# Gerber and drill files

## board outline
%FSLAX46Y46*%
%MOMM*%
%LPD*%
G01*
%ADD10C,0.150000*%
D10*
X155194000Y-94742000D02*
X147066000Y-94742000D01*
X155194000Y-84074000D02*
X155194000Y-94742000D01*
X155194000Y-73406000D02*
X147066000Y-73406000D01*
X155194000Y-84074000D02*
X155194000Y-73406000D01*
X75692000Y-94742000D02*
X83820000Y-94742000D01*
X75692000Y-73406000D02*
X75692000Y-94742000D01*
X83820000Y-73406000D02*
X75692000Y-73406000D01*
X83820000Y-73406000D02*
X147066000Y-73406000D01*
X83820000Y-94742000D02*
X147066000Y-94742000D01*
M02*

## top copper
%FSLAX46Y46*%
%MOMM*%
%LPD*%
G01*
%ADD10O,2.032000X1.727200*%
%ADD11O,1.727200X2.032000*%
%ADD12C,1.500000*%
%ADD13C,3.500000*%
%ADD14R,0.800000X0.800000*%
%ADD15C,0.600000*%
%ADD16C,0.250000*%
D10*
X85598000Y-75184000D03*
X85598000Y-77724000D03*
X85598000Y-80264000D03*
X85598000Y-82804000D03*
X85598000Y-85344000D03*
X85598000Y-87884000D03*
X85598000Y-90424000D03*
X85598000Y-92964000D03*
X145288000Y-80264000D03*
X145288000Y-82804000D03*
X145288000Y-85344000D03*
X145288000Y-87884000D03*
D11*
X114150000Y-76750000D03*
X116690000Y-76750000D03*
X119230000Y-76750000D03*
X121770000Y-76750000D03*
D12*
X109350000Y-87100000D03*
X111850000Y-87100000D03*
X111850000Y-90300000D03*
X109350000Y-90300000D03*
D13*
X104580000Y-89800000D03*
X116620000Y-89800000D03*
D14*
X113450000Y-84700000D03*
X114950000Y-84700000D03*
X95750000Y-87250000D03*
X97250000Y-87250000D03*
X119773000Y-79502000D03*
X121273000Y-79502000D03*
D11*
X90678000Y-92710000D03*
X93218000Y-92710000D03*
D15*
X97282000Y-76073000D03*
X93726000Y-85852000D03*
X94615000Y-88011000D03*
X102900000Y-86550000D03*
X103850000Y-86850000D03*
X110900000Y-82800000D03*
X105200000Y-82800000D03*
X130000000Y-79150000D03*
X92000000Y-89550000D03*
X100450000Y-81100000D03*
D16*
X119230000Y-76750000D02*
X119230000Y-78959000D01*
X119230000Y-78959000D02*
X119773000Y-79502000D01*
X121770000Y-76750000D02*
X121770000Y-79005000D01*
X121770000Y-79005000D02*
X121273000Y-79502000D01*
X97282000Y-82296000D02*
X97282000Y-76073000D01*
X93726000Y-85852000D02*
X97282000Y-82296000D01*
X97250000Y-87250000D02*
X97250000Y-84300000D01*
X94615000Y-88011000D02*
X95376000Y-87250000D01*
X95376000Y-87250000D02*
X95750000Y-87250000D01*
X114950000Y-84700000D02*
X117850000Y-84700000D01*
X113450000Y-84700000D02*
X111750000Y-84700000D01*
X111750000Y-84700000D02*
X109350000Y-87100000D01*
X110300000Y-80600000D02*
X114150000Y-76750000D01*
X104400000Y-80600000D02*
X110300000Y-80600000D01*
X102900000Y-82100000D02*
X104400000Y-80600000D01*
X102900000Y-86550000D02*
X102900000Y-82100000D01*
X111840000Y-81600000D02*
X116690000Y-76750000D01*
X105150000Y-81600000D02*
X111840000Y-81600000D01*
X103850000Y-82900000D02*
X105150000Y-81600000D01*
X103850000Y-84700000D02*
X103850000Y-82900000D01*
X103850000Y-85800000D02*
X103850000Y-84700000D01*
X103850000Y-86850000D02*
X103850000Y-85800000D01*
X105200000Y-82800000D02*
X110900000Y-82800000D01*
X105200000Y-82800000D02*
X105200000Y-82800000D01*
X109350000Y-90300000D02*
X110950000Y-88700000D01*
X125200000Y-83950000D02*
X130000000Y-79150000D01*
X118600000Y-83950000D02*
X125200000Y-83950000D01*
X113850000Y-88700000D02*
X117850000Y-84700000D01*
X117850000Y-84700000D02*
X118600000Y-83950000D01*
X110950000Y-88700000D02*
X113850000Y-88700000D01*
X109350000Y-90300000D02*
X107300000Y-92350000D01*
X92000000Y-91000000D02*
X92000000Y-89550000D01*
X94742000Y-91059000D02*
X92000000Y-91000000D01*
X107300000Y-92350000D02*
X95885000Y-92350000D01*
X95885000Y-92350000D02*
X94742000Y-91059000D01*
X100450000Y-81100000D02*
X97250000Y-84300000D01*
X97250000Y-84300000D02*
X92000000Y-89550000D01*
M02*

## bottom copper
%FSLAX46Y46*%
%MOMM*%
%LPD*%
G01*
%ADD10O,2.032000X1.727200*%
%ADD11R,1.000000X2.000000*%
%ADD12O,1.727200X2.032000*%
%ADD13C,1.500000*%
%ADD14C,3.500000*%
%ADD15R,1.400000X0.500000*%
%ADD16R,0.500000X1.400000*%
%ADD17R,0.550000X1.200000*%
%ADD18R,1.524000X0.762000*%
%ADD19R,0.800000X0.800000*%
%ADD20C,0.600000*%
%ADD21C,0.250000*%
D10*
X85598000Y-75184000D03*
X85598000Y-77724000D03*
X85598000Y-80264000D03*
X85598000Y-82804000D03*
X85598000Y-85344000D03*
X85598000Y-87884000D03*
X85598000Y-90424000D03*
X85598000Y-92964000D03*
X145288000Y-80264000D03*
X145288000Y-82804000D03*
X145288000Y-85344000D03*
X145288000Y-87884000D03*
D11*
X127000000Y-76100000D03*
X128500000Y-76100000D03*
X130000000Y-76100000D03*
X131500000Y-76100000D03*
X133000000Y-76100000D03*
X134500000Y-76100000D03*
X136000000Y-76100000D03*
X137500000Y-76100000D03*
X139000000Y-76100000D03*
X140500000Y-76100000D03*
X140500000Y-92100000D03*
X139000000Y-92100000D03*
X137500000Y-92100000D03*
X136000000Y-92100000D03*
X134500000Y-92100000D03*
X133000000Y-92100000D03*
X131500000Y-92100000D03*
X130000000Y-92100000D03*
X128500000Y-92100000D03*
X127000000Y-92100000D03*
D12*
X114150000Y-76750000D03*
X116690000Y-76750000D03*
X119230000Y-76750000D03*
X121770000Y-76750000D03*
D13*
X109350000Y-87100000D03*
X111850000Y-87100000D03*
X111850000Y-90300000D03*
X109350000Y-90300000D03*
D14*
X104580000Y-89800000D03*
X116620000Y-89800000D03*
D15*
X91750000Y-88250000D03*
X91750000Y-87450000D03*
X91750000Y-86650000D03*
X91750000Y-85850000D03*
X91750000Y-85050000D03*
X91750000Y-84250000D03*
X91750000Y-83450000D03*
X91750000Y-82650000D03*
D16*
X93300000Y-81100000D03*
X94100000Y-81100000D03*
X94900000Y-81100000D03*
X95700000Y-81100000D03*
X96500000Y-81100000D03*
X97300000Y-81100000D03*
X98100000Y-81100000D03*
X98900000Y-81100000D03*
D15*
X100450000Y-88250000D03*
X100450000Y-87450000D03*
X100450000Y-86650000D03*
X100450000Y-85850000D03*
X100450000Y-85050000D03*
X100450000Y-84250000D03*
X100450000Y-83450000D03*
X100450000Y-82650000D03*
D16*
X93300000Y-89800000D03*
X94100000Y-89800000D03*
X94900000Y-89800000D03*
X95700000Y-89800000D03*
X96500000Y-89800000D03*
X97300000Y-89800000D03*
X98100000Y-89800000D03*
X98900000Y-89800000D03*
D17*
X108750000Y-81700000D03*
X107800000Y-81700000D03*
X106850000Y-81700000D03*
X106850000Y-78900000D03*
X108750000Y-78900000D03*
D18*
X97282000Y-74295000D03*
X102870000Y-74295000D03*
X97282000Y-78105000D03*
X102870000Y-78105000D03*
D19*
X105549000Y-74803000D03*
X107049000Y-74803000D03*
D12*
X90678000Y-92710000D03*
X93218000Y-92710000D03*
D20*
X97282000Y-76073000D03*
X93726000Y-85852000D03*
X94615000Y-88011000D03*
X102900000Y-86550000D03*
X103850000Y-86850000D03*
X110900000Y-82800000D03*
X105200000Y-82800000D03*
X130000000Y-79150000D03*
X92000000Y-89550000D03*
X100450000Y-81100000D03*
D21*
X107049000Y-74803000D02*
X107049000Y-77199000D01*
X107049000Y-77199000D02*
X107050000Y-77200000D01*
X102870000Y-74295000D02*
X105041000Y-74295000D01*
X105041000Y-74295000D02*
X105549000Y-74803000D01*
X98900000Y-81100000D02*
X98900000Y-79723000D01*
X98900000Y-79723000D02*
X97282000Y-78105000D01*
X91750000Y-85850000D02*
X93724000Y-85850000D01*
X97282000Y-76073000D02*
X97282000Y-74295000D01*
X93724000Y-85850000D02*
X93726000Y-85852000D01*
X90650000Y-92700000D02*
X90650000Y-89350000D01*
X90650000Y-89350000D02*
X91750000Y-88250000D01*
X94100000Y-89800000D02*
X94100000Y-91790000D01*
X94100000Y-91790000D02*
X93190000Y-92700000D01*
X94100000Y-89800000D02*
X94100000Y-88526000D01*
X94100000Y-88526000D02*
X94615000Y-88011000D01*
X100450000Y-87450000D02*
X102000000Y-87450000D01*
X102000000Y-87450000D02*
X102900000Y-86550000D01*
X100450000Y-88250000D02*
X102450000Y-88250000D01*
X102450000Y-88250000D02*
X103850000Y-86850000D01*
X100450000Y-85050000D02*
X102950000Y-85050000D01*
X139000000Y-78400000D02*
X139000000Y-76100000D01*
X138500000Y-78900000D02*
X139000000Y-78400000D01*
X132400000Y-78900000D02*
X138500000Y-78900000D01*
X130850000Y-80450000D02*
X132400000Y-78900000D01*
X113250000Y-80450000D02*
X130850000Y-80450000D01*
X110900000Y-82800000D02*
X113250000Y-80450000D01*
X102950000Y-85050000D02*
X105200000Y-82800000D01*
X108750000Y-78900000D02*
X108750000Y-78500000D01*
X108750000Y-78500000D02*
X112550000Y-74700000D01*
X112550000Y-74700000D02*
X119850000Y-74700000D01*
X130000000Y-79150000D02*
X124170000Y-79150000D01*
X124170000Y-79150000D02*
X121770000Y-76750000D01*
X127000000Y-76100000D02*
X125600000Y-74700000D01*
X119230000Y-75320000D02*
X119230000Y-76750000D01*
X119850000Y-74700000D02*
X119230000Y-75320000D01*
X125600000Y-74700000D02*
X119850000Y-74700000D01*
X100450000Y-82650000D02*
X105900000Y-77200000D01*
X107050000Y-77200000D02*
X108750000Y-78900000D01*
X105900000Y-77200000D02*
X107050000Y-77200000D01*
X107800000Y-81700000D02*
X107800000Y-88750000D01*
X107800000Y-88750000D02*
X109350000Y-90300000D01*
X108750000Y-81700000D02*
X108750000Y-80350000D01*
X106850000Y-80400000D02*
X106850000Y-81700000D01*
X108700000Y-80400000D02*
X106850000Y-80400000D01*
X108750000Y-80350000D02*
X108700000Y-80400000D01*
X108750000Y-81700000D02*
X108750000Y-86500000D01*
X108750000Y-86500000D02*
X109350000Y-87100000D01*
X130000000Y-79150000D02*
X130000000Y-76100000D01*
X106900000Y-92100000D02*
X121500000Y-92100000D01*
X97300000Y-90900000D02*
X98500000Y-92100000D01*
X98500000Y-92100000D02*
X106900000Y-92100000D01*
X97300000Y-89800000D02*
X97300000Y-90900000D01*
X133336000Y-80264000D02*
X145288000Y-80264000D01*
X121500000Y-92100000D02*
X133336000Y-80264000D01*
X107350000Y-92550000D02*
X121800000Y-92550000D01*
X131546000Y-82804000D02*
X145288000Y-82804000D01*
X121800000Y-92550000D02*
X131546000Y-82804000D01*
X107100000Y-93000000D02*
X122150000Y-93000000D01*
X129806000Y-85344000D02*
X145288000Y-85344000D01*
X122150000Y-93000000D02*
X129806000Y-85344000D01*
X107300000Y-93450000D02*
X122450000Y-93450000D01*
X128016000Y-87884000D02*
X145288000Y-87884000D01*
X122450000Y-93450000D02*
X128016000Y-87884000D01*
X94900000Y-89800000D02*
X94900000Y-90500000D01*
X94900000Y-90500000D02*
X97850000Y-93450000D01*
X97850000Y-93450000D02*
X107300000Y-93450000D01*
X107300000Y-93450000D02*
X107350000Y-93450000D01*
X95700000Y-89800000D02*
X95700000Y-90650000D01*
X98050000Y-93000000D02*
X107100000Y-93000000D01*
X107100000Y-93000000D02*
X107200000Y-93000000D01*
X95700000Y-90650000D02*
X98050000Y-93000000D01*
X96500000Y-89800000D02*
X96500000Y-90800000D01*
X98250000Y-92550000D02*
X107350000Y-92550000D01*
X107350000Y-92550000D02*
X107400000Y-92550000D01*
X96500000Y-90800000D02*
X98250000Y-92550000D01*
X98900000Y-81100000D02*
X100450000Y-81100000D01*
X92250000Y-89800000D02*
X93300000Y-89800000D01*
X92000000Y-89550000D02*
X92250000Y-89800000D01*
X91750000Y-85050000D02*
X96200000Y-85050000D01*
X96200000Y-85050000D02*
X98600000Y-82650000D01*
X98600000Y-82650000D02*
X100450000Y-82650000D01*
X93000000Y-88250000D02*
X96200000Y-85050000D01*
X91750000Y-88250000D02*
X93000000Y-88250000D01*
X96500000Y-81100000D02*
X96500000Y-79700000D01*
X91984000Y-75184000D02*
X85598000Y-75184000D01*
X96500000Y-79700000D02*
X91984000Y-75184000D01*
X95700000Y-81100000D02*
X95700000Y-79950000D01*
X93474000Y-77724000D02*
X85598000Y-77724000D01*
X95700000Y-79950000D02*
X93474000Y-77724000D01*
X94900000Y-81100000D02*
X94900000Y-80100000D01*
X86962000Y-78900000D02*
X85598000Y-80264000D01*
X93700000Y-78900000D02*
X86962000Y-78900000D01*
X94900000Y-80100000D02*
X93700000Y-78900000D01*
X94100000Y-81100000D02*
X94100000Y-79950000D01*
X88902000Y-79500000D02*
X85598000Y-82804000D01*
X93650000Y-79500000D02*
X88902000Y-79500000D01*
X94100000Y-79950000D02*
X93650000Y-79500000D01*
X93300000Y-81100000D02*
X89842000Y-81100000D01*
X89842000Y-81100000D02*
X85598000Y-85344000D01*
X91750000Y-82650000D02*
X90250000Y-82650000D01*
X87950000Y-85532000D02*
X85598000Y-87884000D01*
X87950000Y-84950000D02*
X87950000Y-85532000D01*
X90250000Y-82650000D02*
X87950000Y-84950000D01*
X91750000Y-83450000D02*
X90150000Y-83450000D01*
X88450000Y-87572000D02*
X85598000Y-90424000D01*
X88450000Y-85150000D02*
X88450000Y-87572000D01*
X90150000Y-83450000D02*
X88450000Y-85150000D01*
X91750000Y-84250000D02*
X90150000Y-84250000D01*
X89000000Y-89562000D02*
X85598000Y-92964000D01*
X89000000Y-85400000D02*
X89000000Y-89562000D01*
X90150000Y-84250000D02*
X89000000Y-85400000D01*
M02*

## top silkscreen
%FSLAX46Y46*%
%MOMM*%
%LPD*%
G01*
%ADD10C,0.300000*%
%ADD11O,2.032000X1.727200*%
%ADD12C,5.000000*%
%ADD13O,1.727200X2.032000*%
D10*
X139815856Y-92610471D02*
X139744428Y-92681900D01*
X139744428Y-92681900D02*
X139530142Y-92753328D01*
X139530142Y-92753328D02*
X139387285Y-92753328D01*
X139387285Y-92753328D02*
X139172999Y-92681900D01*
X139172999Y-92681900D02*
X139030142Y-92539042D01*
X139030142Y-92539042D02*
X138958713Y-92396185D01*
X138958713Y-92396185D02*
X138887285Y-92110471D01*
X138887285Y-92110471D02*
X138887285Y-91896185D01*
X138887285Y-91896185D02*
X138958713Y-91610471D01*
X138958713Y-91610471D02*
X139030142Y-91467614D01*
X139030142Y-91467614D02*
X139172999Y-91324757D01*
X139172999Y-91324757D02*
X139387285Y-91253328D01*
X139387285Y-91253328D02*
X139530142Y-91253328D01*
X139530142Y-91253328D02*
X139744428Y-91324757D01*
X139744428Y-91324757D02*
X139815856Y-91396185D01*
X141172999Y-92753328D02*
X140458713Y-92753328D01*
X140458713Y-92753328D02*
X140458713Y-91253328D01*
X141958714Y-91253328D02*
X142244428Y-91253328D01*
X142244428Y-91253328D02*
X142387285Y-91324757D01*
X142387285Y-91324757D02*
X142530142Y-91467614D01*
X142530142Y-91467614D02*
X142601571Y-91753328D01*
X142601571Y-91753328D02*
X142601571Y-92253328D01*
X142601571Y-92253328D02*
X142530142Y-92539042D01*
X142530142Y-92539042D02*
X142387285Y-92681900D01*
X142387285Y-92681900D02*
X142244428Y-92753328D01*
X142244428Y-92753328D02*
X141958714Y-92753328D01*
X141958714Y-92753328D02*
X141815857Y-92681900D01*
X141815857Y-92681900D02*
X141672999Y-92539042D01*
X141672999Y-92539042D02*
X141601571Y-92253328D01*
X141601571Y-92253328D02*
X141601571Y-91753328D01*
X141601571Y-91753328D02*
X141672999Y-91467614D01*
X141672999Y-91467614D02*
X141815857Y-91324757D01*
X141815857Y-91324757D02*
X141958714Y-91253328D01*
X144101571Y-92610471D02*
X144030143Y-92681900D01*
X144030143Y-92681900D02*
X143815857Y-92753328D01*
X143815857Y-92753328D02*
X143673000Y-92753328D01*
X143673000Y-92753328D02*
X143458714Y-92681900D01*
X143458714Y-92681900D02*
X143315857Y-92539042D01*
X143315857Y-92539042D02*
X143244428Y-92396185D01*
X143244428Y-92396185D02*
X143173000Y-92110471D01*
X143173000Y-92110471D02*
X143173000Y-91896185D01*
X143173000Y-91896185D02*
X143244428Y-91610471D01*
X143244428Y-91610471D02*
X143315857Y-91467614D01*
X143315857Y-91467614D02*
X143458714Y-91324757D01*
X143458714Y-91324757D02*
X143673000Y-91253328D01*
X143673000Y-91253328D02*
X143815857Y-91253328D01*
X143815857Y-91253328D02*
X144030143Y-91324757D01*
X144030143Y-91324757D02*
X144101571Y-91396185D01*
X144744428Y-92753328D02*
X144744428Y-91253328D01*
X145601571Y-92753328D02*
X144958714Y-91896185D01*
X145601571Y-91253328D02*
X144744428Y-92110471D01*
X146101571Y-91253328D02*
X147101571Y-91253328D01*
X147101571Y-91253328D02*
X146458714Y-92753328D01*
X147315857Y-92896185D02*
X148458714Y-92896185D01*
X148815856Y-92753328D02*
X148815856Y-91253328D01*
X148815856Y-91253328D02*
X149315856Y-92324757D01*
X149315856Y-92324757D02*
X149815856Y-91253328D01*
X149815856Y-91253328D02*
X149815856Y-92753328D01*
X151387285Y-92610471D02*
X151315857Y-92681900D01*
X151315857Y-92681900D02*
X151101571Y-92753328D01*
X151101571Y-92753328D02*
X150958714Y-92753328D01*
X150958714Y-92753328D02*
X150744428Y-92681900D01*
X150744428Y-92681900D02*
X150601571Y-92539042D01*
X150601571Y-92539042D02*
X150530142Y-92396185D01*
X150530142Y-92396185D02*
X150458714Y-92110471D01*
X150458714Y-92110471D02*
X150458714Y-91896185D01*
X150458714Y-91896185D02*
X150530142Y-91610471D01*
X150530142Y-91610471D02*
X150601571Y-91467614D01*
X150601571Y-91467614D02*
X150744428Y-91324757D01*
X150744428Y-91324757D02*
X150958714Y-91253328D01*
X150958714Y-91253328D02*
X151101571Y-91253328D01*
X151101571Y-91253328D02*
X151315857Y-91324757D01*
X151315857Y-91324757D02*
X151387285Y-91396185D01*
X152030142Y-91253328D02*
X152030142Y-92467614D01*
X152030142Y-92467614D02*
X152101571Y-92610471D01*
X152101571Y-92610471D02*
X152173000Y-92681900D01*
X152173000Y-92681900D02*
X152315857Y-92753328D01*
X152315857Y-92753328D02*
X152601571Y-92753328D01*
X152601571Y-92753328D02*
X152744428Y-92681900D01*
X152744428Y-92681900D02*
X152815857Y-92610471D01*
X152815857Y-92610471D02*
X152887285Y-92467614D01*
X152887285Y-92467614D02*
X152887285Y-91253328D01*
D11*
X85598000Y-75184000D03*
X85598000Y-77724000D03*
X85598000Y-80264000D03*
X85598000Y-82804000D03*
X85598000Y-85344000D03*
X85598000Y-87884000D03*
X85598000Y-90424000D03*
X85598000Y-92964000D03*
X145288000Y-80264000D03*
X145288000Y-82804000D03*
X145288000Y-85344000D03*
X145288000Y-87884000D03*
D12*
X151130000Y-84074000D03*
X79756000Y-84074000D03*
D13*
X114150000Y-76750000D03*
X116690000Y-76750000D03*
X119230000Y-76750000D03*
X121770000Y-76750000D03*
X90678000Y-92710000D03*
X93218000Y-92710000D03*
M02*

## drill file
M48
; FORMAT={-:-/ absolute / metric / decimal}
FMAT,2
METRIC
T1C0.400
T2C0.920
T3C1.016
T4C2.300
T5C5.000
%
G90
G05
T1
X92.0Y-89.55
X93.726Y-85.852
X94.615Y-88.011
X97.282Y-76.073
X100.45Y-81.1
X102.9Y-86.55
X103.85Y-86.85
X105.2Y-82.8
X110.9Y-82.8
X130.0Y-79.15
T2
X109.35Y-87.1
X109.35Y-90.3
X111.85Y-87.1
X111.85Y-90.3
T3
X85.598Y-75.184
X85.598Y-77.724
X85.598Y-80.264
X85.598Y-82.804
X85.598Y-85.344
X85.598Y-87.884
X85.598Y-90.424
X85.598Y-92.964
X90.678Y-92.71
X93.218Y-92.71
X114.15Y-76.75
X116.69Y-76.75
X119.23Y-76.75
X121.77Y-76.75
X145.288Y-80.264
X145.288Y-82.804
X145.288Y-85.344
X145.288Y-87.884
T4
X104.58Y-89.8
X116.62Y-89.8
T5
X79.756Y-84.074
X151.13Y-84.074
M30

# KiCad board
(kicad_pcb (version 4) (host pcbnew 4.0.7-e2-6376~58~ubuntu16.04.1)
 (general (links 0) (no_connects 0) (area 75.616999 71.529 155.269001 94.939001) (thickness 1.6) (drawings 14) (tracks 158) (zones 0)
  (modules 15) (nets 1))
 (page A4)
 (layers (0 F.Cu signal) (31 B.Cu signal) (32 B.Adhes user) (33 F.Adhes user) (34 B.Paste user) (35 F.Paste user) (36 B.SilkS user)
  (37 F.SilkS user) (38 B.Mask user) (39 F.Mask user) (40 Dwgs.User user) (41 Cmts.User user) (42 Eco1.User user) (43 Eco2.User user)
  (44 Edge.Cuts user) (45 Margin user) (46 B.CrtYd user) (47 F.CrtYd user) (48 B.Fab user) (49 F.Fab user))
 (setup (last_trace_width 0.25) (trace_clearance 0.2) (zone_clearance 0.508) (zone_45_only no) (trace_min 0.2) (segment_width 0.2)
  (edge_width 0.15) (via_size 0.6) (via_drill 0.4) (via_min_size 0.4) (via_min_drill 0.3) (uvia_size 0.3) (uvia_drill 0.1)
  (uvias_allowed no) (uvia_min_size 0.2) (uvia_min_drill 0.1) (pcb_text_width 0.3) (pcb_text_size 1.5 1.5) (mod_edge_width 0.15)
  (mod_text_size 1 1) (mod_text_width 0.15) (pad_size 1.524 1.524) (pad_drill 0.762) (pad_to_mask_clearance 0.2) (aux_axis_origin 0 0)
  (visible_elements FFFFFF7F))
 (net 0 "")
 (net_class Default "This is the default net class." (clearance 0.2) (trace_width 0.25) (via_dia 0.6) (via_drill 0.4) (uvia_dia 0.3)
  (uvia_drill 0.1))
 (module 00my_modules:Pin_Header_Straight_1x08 (layer F.Cu) (at 85.598 75.184)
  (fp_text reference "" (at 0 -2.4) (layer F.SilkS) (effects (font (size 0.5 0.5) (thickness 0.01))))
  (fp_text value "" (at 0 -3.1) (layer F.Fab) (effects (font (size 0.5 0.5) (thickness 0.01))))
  (pad 1 thru_hole oval (at 0 0) (size 2.032 1.7272) (drill 1.016) (layers *.Cu *.Mask F.SilkS))
  (pad 2 thru_hole oval (at 0 2.54) (size 2.032 1.7272) (drill 1.016) (layers *.Cu *.Mask F.SilkS))
  (pad 3 thru_hole oval (at 0 5.08) (size 2.032 1.7272) (drill 1.016) (layers *.Cu *.Mask F.SilkS))
  (pad 4 thru_hole oval (at 0 7.62) (size 2.032 1.7272) (drill 1.016) (layers *.Cu *.Mask F.SilkS))
  (pad 5 thru_hole oval (at 0 10.16) (size 2.032 1.7272) (drill 1.016) (layers *.Cu *.Mask F.SilkS))
  (pad 6 thru_hole oval (at 0 12.7) (size 2.032 1.7272) (drill 1.016) (layers *.Cu *.Mask F.SilkS))
  (pad 7 thru_hole oval (at 0 15.24) (size 2.032 1.7272) (drill 1.016) (layers *.Cu *.Mask F.SilkS))
  (pad 8 thru_hole oval (at 0 17.78) (size 2.032 1.7272) (drill 1.016) (layers *.Cu *.Mask F.SilkS)))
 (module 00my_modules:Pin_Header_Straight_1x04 (layer F.Cu) (at 145.288 80.264)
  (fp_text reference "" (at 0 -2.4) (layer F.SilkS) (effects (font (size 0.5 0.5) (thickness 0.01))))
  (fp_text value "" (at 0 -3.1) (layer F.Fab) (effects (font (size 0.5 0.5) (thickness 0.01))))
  (pad 1 thru_hole oval (at 0 0) (size 2.032 1.7272) (drill 1.016) (layers *.Cu *.Mask F.SilkS))
  (pad 2 thru_hole oval (at 0 2.54) (size 2.032 1.7272) (drill 1.016) (layers *.Cu *.Mask F.SilkS))
  (pad 3 thru_hole oval (at 0 5.08) (size 2.032 1.7272) (drill 1.016) (layers *.Cu *.Mask F.SilkS))
  (pad 4 thru_hole oval (at 0 7.62) (size 2.032 1.7272) (drill 1.016) (layers *.Cu *.Mask F.SilkS)))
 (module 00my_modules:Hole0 (layer F.Cu) (at 151.13 84.074)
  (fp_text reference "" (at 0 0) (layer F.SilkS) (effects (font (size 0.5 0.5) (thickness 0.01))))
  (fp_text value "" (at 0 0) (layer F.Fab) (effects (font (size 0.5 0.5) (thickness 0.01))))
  (pad "" np_thru_hole circle (at 0 0) (size 5 5) (drill 5) (layers *.Cu *.Mask F.SilkS)))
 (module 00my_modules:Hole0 (layer F.Cu) (at 79.756 84.074)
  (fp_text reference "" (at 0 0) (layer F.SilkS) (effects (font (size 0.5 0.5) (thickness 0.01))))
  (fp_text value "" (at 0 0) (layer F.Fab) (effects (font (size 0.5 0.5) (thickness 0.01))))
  (pad "" np_thru_hole circle (at 0 0) (size 5 5) (drill 5) (layers *.Cu *.Mask F.SilkS)))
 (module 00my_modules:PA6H (layer B.Cu) (at 133.75 84.1 270)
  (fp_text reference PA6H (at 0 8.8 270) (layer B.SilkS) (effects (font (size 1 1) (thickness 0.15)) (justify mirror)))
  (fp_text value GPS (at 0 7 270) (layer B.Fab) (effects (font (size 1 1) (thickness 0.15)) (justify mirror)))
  (pad VCC smd rect (at -8 6.75 270) (size 2 1) (layers B.Cu B.Paste B.Mask))
  (pad 2 smd rect (at -8 5.25 270) (size 2 1) (layers B.Cu B.Paste B.Mask))
  (pad GND smd rect (at -8 3.75 270) (size 2 1) (layers B.Cu B.Paste B.Mask))
  (pad 4 smd rect (at -8 2.25 270) (size 2 1) (layers B.Cu B.Paste B.Mask))
  (pad 5 smd rect (at -8 0.75 270) (size 2 1) (layers B.Cu B.Paste B.Mask))
  (pad 6 smd rect (at -8 -0.75 270) (size 2 1) (layers B.Cu B.Paste B.Mask))
  (pad 7 smd rect (at -8 -2.25 270) (size 2 1) (layers B.Cu B.Paste B.Mask))
  (pad 8 smd rect (at -8 -3.75 270) (size 2 1) (layers B.Cu B.Paste B.Mask))
  (pad TX smd rect (at -8 -5.25 270) (size 2 1) (layers B.Cu B.Paste B.Mask))
  (pad RX smd rect (at -8 -6.75 270) (size 2 1) (layers B.Cu B.Paste B.Mask))
  (pad 11 smd rect (at 8 -6.75 270) (size 2 1) (layers B.Cu B.Paste B.Mask))
  (pad 12 smd rect (at 8 -5.25 270) (size 2 1) (layers B.Cu B.Paste B.Mask))
  (pad 13 smd rect (at 8 -3.75 270) (size 2 1) (layers B.Cu B.Paste B.Mask))
  (pad 14 smd rect (at 8 -2.25 270) (size 2 1) (layers B.Cu B.Paste B.Mask))
  (pad 15 smd rect (at 8 -0.75 270) (size 2 1) (layers B.Cu B.Paste B.Mask))
  (pad 16 smd rect (at 8 0.75 270) (size 2 1) (layers B.Cu B.Paste B.Mask))
  (pad 17 smd rect (at 8 2.25 270) (size 2 1) (layers B.Cu B.Paste B.Mask))
  (pad 18 smd rect (at 8 3.75 270) (size 2 1) (layers B.Cu B.Paste B.Mask))
  (pad 19 smd rect (at 8 5.25 270) (size 2 1) (layers B.Cu B.Paste B.Mask))
  (pad 20 smd rect (at 8 6.75 270) (size 2 1) (layers B.Cu B.Paste B.Mask)))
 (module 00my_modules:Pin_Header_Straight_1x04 (layer F.Cu) (at 114.15 76.75 90)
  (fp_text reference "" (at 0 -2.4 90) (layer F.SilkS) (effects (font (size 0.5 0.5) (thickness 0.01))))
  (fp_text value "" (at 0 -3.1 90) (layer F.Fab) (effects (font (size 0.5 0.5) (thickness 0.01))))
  (pad 1 thru_hole oval (at 0 0 90) (size 2.032 1.7272) (drill 1.016) (layers *.Cu *.Mask F.SilkS))
  (pad 2 thru_hole oval (at 0 2.54 90) (size 2.032 1.7272) (drill 1.016) (layers *.Cu *.Mask F.SilkS))
  (pad 3 thru_hole oval (at 0 5.08 90) (size 2.032 1.7272) (drill 1.016) (layers *.Cu *.Mask F.SilkS))
  (pad 4 thru_hole oval (at 0 7.62 90) (size 2.032 1.7272) (drill 1.016) (layers *.Cu *.Mask F.SilkS)))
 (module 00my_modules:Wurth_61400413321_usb (layer B.Cu) (at 110.6 89.8 180)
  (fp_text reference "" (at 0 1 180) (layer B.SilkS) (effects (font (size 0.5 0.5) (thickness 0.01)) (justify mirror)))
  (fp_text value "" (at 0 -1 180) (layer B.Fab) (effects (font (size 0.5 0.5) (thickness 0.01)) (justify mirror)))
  (pad V thru_hole circle (at 1.25 2.7 180) (size 1.5 1.5) (drill 0.92) (layers *.Cu *.Mask B.SilkS))
  (pad - thru_hole circle (at -1.25 2.7 180) (size 1.5 1.5) (drill 0.92) (layers *.Cu *.Mask B.SilkS))
  (pad + thru_hole circle (at -1.25 -0.5 180) (size 1.5 1.5) (drill 0.92) (layers *.Cu *.Mask B.SilkS))
  (pad G thru_hole circle (at 1.25 -0.5 180) (size 1.5 1.5) (drill 0.92) (layers *.Cu *.Mask B.SilkS))
  (pad X thru_hole circle (at 6.02 0 180) (size 3.5 3.5) (drill 2.3) (layers *.Cu *.Mask B.SilkS))
  (pad X thru_hole circle (at -6.02 0 180) (size 3.5 3.5) (drill 2.3) (layers *.Cu *.Mask B.SilkS)))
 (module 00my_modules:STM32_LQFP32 (layer B.Cu) (at 96.1 85.45)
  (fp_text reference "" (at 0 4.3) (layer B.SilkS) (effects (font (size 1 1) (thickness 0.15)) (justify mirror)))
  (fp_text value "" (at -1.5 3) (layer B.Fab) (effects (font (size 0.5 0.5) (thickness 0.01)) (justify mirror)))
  (pad 3.3 smd rect (at -4.35 2.8) (size 1.4 0.5) (layers B.Cu B.Paste B.Mask))
  (pad PF0 smd rect (at -4.35 2) (size 1.4 0.5) (layers B.Cu B.Paste B.Mask))
  (pad PF1 smd rect (at -4.35 1.2) (size 1.4 0.5) (layers B.Cu B.Paste B.Mask))
  (pad RST smd rect (at -4.35 0.4) (size 1.4 0.5) (layers B.Cu B.Paste B.Mask))
  (pad 3.3 smd rect (at -4.35 -0.4) (size 1.4 0.5) (layers B.Cu B.Paste B.Mask))
  (pad PA0 smd rect (at -4.35 -1.2) (size 1.4 0.5) (layers B.Cu B.Paste B.Mask))
  (pad PA1 smd rect (at -4.35 -2) (size 1.4 0.5) (layers B.Cu B.Paste B.Mask))
  (pad PA2 smd rect (at -4.35 -2.8) (size 1.4 0.5) (layers B.Cu B.Paste B.Mask))
  (pad PA3 smd rect (at -2.8 -4.35 270) (size 1.4 0.5) (layers B.Cu B.Paste B.Mask))
  (pad PA4 smd rect (at -2 -4.35 270) (size 1.4 0.5) (layers B.Cu B.Paste B.Mask))
  (pad PA5 smd rect (at -1.2 -4.35 270) (size 1.4 0.5) (layers B.Cu B.Paste B.Mask))
  (pad PA6 smd rect (at -0.4 -4.35 270) (size 1.4 0.5) (layers B.Cu B.Paste B.Mask))
  (pad PA7 smd rect (at 0.4 -4.35 270) (size 1.4 0.5) (layers B.Cu B.Paste B.Mask))
  (pad PB0 smd rect (at 1.2 -4.35 270) (size 1.4 0.5) (layers B.Cu B.Paste B.Mask))
  (pad PB1 smd rect (at 2 -4.35 270) (size 1.4 0.5) (layers B.Cu B.Paste B.Mask))
  (pad GND smd rect (at 2.8 -4.35 270) (size 1.4 0.5) (layers B.Cu B.Paste B.Mask))
  (pad PA14 smd rect (at 4.35 2.8) (size 1.4 0.5) (layers B.Cu B.Paste B.Mask))
  (pad PA13 smd rect (at 4.35 2) (size 1.4 0.5) (layers B.Cu B.Paste B.Mask))
  (pad PA12 smd rect (at 4.35 1.2) (size 1.4 0.5) (layers B.Cu B.Paste B.Mask))
  (pad PA11 smd rect (at 4.35 0.4) (size 1.4 0.5) (layers B.Cu B.Paste B.Mask))
  (pad PA10 smd rect (at 4.35 -0.4) (size 1.4 0.5) (layers B.Cu B.Paste B.Mask))
  (pad PA9 smd rect (at 4.35 -1.2) (size 1.4 0.5) (layers B.Cu B.Paste B.Mask))
  (pad PA8 smd rect (at 4.35 -2) (size 1.4 0.5) (layers B.Cu B.Paste B.Mask))
  (pad 3.3 smd rect (at 4.35 -2.8) (size 1.4 0.5) (layers B.Cu B.Paste B.Mask))
  (pad GND smd rect (at -2.8 4.35 270) (size 1.4 0.5) (layers B.Cu B.Paste B.Mask))
  (pad BOOT smd rect (at -2 4.35 270) (size 1.4 0.5) (layers B.Cu B.Paste B.Mask))
  (pad PB7 smd rect (at -1.2 4.35 270) (size 1.4 0.5) (layers B.Cu B.Paste B.Mask))
  (pad PB6 smd rect (at -0.4 4.35 270) (size 1.4 0.5) (layers B.Cu B.Paste B.Mask))
  (pad PB5 smd rect (at 0.4 4.35 270) (size 1.4 0.5) (layers B.Cu B.Paste B.Mask))
  (pad PB4 smd rect (at 1.2 4.35 270) (size 1.4 0.5) (layers B.Cu B.Paste B.Mask))
  (pad PB3 smd rect (at 2 4.35 270) (size 1.4 0.5) (layers B.Cu B.Paste B.Mask))
  (pad PA15 smd rect (at 2.8 4.35 270) (size 1.4 0.5) (layers B.Cu B.Paste B.Mask)))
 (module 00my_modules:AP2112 (layer B.Cu) (at 107.8 80.3 90)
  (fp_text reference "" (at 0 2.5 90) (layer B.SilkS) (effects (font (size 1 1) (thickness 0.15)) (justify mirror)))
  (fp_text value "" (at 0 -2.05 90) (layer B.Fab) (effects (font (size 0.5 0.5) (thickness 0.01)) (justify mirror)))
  (pad VIN smd rect (at -1.4 0.95 90) (size 1.2 0.55) (layers B.Cu B.Paste B.Mask))
  (pad GND smd rect (at -1.4 0 90) (size 1.2 0.55) (layers B.Cu B.Paste B.Mask))
  (pad EN smd rect (at -1.4 -0.95 90) (size 1.2 0.55) (layers B.Cu B.Paste B.Mask))
  (pad NC smd rect (at 1.4 -0.95 90) (size 1.2 0.55) (layers B.Cu B.Paste B.Mask))
  (pad VOUT smd rect (at 1.4 0.95 90) (size 1.2 0.55) (layers B.Cu B.Paste B.Mask)))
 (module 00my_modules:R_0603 (layer F.Cu) (at 114.2 84.7)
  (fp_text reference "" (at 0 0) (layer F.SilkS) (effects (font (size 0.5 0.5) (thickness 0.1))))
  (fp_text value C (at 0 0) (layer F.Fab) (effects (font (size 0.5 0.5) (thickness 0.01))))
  (pad 1 smd rect (at -0.75 0) (size 0.8 0.8) (layers F.Cu F.Paste F.Mask))
  (pad 2 smd rect (at 0.75 0) (size 0.8 0.8) (layers F.Cu F.Paste F.Mask)))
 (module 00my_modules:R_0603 (layer F.Cu) (at 96.5 87.25)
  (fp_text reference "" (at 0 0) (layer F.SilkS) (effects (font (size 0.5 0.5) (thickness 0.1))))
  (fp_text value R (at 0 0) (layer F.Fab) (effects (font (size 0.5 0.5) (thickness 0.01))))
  (pad 1 smd rect (at -0.75 0) (size 0.8 0.8) (layers F.Cu F.Paste F.Mask))
  (pad 2 smd rect (at 0.75 0) (size 0.8 0.8) (layers F.Cu F.Paste F.Mask)))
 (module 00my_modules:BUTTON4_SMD (layer B.Cu) (at 100.076 76.2)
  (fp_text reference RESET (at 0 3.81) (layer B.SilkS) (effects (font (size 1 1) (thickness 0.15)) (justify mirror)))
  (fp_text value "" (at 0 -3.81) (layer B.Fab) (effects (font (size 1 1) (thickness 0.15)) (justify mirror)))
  (pad 1 smd rect (at -2.794 -1.905) (size 1.524 0.762) (layers B.Cu B.Paste B.Mask))
  (pad 2 smd rect (at 2.794 -1.905) (size 1.524 0.762) (layers B.Cu B.Paste B.Mask))
  (pad 3 smd rect (at -2.794 1.905) (size 1.524 0.762) (layers B.Cu B.Paste B.Mask))
  (pad 4 smd rect (at 2.794 1.905) (size 1.524 0.762) (layers B.Cu B.Paste B.Mask)))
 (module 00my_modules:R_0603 (layer B.Cu) (at 106.299 74.803)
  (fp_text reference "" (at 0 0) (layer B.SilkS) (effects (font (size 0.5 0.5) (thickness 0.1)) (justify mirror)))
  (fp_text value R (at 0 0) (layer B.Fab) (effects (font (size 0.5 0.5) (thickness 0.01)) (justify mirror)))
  (pad 1 smd rect (at -0.75 0) (size 0.8 0.8) (layers B.Cu B.Paste B.Mask))
  (pad 2 smd rect (at 0.75 0) (size 0.8 0.8) (layers B.Cu B.Paste B.Mask)))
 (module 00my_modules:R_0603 (layer F.Cu) (at 120.523 79.502)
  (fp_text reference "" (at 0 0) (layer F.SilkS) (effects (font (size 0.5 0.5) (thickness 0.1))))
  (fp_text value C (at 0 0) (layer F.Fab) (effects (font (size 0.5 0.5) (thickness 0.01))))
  (pad 1 smd rect (at -0.75 0) (size 0.8 0.8) (layers F.Cu F.Paste F.Mask))
  (pad 2 smd rect (at 0.75 0) (size 0.8 0.8) (layers F.Cu F.Paste F.Mask)))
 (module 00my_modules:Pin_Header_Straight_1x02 (layer F.Cu) (at 90.678 92.71 90)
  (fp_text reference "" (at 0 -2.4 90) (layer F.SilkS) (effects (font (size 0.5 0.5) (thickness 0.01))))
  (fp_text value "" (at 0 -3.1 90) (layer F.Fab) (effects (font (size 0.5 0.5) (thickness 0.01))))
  (pad 1 thru_hole oval (at 0 0 90) (size 2.032 1.7272) (drill 1.016) (layers *.Cu *.Mask F.SilkS))
  (pad 2 thru_hole oval (at 0 2.54 90) (size 2.032 1.7272) (drill 1.016) (layers *.Cu *.Mask F.SilkS)))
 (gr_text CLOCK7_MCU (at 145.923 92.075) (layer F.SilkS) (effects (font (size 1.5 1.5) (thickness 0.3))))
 (gr_line (start 155.194 94.742) (end 147.066 94.742) (angle 90) (layer Edge.Cuts) (width 0.15))
 (gr_line (start 155.194 84.074) (end 155.194 94.742) (angle 90) (layer Edge.Cuts) (width 0.15))
 (gr_line (start 155.194 73.406) (end 147.066 73.406) (angle 90) (layer Edge.Cuts) (width 0.15))
 (gr_line (start 155.194 84.074) (end 155.194 73.406) (angle 90) (layer Edge.Cuts) (width 0.15))
 (gr_line (start 75.692 94.742) (end 83.82 94.742) (angle 90) (layer Edge.Cuts) (width 0.15))
 (gr_line (start 75.692 73.406) (end 75.692 94.742) (angle 90) (layer Edge.Cuts) (width 0.15))
 (gr_line (start 83.82 73.406) (end 75.692 73.406) (angle 90) (layer Edge.Cuts) (width 0.15))
 (gr_line (start 83.82 73.406) (end 147.066 73.406) (angle 90) (layer Edge.Cuts) (width 0.15))
 (gr_line (start 83.82 94.742) (end 147.066 94.742) (angle 90) (layer Edge.Cuts) (width 0.15))
 (segment (start 119.23 76.75) (end 119.23 78.959) (width 0.25) (layer F.Cu) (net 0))
 (segment (start 119.23 78.959) (end 119.773 79.502) (width 0.25) (layer F.Cu) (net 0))
 (segment (start 121.77 76.75) (end 121.77 79.005) (width 0.25) (layer F.Cu) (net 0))
 (segment (start 121.77 79.005) (end 121.273 79.502) (width 0.25) (layer F.Cu) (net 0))
 (segment (start 107.049 74.803) (end 107.049 77.199) (width 0.25) (layer B.Cu) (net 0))
 (segment (start 107.049 77.199) (end 107.05 77.2) (width 0.25) (layer B.Cu) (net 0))
 (segment (start 102.87 74.295) (end 105.041 74.295) (width 0.25) (layer B.Cu) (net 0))
 (segment (start 105.041 74.295) (end 105.549 74.803) (width 0.25) (layer B.Cu) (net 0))
 (segment (start 98.9 81.1) (end 98.9 79.723) (width 0.25) (layer B.Cu) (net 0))
 (segment (start 98.9 79.723) (end 97.282 78.105) (width 0.25) (layer B.Cu) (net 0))
 (segment (start 91.75 85.85) (end 93.724 85.85) (width 0.25) (layer B.Cu) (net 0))
 (segment (start 97.282 76.073) (end 97.282 74.295) (width 0.25) (layer B.Cu) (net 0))
 (via (at 97.282 76.073) (size 0.6) (drill 0.4) (layers F.Cu B.Cu) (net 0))
 (segment (start 97.282 82.296) (end 97.282 76.073) (width 0.25) (layer F.Cu) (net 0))
 (segment (start 93.726 85.852) (end 97.282 82.296) (width 0.25) (layer F.Cu) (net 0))
 (via (at 93.726 85.852) (size 0.6) (drill 0.4) (layers F.Cu B.Cu) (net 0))
 (segment (start 93.724 85.85) (end 93.726 85.852) (width 0.25) (layer B.Cu) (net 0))
 (segment (start 90.65 92.7) (end 90.65 89.35) (width 0.25) (layer B.Cu) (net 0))
 (segment (start 90.65 89.35) (end 91.75 88.25) (width 0.25) (layer B.Cu) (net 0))
 (segment (start 94.1 89.8) (end 94.1 91.79) (width 0.25) (layer B.Cu) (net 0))
 (segment (start 94.1 91.79) (end 93.19 92.7) (width 0.25) (layer B.Cu) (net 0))
 (segment (start 97.25 87.25) (end 97.25 84.3) (width 0.25) (layer F.Cu) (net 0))
 (segment (start 94.1 89.8) (end 94.1 88.526) (width 0.25) (layer B.Cu) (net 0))
 (segment (start 94.615 88.011) (end 95.376 87.25) (width 0.25) (layer F.Cu) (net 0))
 (via (at 94.615 88.011) (size 0.6) (drill 0.4) (layers F.Cu B.Cu) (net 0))
 (segment (start 94.1 88.526) (end 94.615 88.011) (width 0.25) (layer B.Cu) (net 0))
 (segment (start 95.376 87.25) (end 95.75 87.25) (width 0.25) (layer F.Cu) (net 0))
 (segment (start 114.95 84.7) (end 117.85 84.7) (width 0.25) (layer F.Cu) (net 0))
 (segment (start 113.45 84.7) (end 111.75 84.7) (width 0.25) (layer F.Cu) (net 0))
 (segment (start 111.75 84.7) (end 109.35 87.1) (width 0.25) (layer F.Cu) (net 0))
 (segment (start 100.45 87.45) (end 102 87.45) (width 0.25) (layer B.Cu) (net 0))
 (segment (start 110.3 80.6) (end 114.15 76.75) (width 0.25) (layer F.Cu) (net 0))
 (segment (start 104.4 80.6) (end 110.3 80.6) (width 0.25) (layer F.Cu) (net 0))
 (segment (start 102.9 82.1) (end 104.4 80.6) (width 0.25) (layer F.Cu) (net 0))
 (segment (start 102.9 86.55) (end 102.9 82.1) (width 0.25) (layer F.Cu) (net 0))
 (via (at 102.9 86.55) (size 0.6) (drill 0.4) (layers F.Cu B.Cu) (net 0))
 (segment (start 102 87.45) (end 102.9 86.55) (width 0.25) (layer B.Cu) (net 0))
 (segment (start 100.45 88.25) (end 102.45 88.25) (width 0.25) (layer B.Cu) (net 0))
 (segment (start 111.84 81.6) (end 116.69 76.75) (width 0.25) (layer F.Cu) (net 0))
 (segment (start 105.15 81.6) (end 111.84 81.6) (width 0.25) (layer F.Cu) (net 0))
 (segment (start 103.85 82.9) (end 105.15 81.6) (width 0.25) (layer F.Cu) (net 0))
 (segment (start 103.85 84.7) (end 103.85 82.9) (width 0.25) (layer F.Cu) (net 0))
 (segment (start 103.85 85.8) (end 103.85 84.7) (width 0.25) (layer F.Cu) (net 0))
 (segment (start 103.85 86.85) (end 103.85 85.8) (width 0.25) (layer F.Cu) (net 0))
 (via (at 103.85 86.85) (size 0.6) (drill 0.4) (layers F.Cu B.Cu) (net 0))
 (segment (start 102.45 88.25) (end 103.85 86.85) (width 0.25) (layer B.Cu) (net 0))
 (segment (start 100.45 85.05) (end 102.95 85.05) (width 0.25) (layer B.Cu) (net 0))
 (segment (start 139 78.4) (end 139 76.1) (width 0.25) (layer B.Cu) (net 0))
 (segment (start 138.5 78.9) (end 139 78.4) (width 0.25) (layer B.Cu) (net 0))
 (segment (start 132.4 78.9) (end 138.5 78.9) (width 0.25) (layer B.Cu) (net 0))
 (segment (start 130.85 80.45) (end 132.4 78.9) (width 0.25) (layer B.Cu) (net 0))
 (segment (start 113.25 80.45) (end 130.85 80.45) (width 0.25) (layer B.Cu) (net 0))
 (segment (start 110.9 82.8) (end 113.25 80.45) (width 0.25) (layer B.Cu) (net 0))
 (via (at 110.9 82.8) (size 0.6) (drill 0.4) (layers F.Cu B.Cu) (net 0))
 (segment (start 105.2 82.8) (end 110.9 82.8) (width 0.25) (layer F.Cu) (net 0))
 (segment (start 105.2 82.8) (end 105.2 82.8) (width 0.25) (layer F.Cu) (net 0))
 (via (at 105.2 82.8) (size 0.6) (drill 0.4) (layers F.Cu B.Cu) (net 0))
 (segment (start 102.95 85.05) (end 105.2 82.8) (width 0.25) (layer B.Cu) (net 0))
 (segment (start 108.75 78.9) (end 108.75 78.5) (width 0.25) (layer B.Cu) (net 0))
 (segment (start 108.75 78.5) (end 112.55 74.7) (width 0.25) (layer B.Cu) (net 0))
 (segment (start 112.55 74.7) (end 119.85 74.7) (width 0.25) (layer B.Cu) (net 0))
 (segment (start 130 79.15) (end 124.17 79.15) (width 0.25) (layer B.Cu) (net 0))
 (segment (start 124.17 79.15) (end 121.77 76.75) (width 0.25) (layer B.Cu) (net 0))
 (segment (start 127 76.1) (end 125.6 74.7) (width 0.25) (layer B.Cu) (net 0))
 (segment (start 119.23 75.32) (end 119.23 76.75) (width 0.25) (layer B.Cu) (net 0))
 (segment (start 119.85 74.7) (end 119.23 75.32) (width 0.25) (layer B.Cu) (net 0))
 (segment (start 125.6 74.7) (end 119.85 74.7) (width 0.25) (layer B.Cu) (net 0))
 (segment (start 100.45 82.65) (end 105.9 77.2) (width 0.25) (layer B.Cu) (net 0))
 (segment (start 107.05 77.2) (end 108.75 78.9) (width 0.25) (layer B.Cu) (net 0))
 (segment (start 105.9 77.2) (end 107.05 77.2) (width 0.25) (layer B.Cu) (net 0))
 (segment (start 107.8 81.7) (end 107.8 88.75) (width 0.25) (layer B.Cu) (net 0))
 (segment (start 107.8 88.75) (end 109.35 90.3) (width 0.25) (layer B.Cu) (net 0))
 (segment (start 108.75 81.7) (end 108.75 80.35) (width 0.25) (layer B.Cu) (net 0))
 (segment (start 106.85 80.4) (end 106.85 81.7) (width 0.25) (layer B.Cu) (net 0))
 (segment (start 108.7 80.4) (end 106.85 80.4) (width 0.25) (layer B.Cu) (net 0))
 (segment (start 108.75 80.35) (end 108.7 80.4) (width 0.25) (layer B.Cu) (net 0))
 (segment (start 108.75 81.7) (end 108.75 86.5) (width 0.25) (layer B.Cu) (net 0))
 (segment (start 108.75 86.5) (end 109.35 87.1) (width 0.25) (layer B.Cu) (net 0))
 (segment (start 109.35 90.3) (end 110.95 88.7) (width 0.25) (layer F.Cu) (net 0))
 (segment (start 130 79.15) (end 130 76.1) (width 0.25) (layer B.Cu) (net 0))
 (via (at 130 79.15) (size 0.6) (drill 0.4) (layers F.Cu B.Cu) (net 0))
 (segment (start 125.2 83.95) (end 130 79.15) (width 0.25) (layer F.Cu) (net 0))
 (segment (start 118.6 83.95) (end 125.2 83.95) (width 0.25) (layer F.Cu) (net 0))
 (segment (start 113.85 88.7) (end 117.85 84.7) (width 0.25) (layer F.Cu) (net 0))
 (segment (start 117.85 84.7) (end 118.6 83.95) (width 0.25) (layer F.Cu) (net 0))
 (segment (start 110.95 88.7) (end 113.85 88.7) (width 0.25) (layer F.Cu) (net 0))
 (segment (start 109.35 90.3) (end 107.3 92.35) (width 0.25) (layer F.Cu) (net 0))
 (segment (start 92 91) (end 92 89.55) (width 0.25) (layer F.Cu) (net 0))
 (segment (start 94.742 91.059) (end 92 91) (width 0.25) (layer F.Cu) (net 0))
 (segment (start 107.3 92.35) (end 95.885 92.35) (width 0.25) (layer F.Cu) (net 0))
 (segment (start 95.885 92.35) (end 94.742 91.059) (width 0.25) (layer F.Cu) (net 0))
 (segment (start 106.9 92.1) (end 121.5 92.1) (width 0.25) (layer B.Cu) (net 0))
 (segment (start 97.3 90.9) (end 98.5 92.1) (width 0.25) (layer B.Cu) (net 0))
 (segment (start 98.5 92.1) (end 106.9 92.1) (width 0.25) (layer B.Cu) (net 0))
 (segment (start 97.3 89.8) (end 97.3 90.9) (width 0.25) (layer B.Cu) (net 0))
 (segment (start 133.336 80.264) (end 145.288 80.264) (width 0.25) (layer B.Cu) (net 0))
 (segment (start 121.5 92.1) (end 133.336 80.264) (width 0.25) (layer B.Cu) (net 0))
 (segment (start 107.35 92.55) (end 121.8 92.55) (width 0.25) (layer B.Cu) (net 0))
 (segment (start 131.546 82.804) (end 145.288 82.804) (width 0.25) (layer B.Cu) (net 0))
 (segment (start 121.8 92.55) (end 131.546 82.804) (width 0.25) (layer B.Cu) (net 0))
 (segment (start 107.1 93) (end 122.15 93) (width 0.25) (layer B.Cu) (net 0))
 (segment (start 129.806 85.344) (end 145.288 85.344) (width 0.25) (layer B.Cu) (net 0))
 (segment (start 122.15 93) (end 129.806 85.344) (width 0.25) (layer B.Cu) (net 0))
 (segment (start 107.3 93.45) (end 122.45 93.45) (width 0.25) (layer B.Cu) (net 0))
 (segment (start 128.016 87.884) (end 145.288 87.884) (width 0.25) (layer B.Cu) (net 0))
 (segment (start 122.45 93.45) (end 128.016 87.884) (width 0.25) (layer B.Cu) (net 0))
 (segment (start 94.9 89.8) (end 94.9 90.5) (width 0.25) (layer B.Cu) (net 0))
 (segment (start 94.9 90.5) (end 97.85 93.45) (width 0.25) (layer B.Cu) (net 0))
 (segment (start 97.85 93.45) (end 107.3 93.45) (width 0.25) (layer B.Cu) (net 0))
 (segment (start 107.3 93.45) (end 107.35 93.45) (width 0.25) (layer B.Cu) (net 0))
 (segment (start 95.7 89.8) (end 95.7 90.65) (width 0.25) (layer B.Cu) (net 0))
 (segment (start 98.05 93) (end 107.1 93) (width 0.25) (layer B.Cu) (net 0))
 (segment (start 107.1 93) (end 107.2 93) (width 0.25) (layer B.Cu) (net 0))
 (segment (start 95.7 90.65) (end 98.05 93) (width 0.25) (layer B.Cu) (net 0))
 (segment (start 96.5 89.8) (end 96.5 90.8) (width 0.25) (layer B.Cu) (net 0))
 (segment (start 98.25 92.55) (end 107.35 92.55) (width 0.25) (layer B.Cu) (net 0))
 (segment (start 107.35 92.55) (end 107.4 92.55) (width 0.25) (layer B.Cu) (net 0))
 (segment (start 96.5 90.8) (end 98.25 92.55) (width 0.25) (layer B.Cu) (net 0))
 (segment (start 98.9 81.1) (end 100.45 81.1) (width 0.25) (layer B.Cu) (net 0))
 (segment (start 92.25 89.8) (end 93.3 89.8) (width 0.25) (layer B.Cu) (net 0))
 (segment (start 92 89.55) (end 92.25 89.8) (width 0.25) (layer B.Cu) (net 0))
 (via (at 92 89.55) (size 0.6) (drill 0.4) (layers F.Cu B.Cu) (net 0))
 (segment (start 100.45 81.1) (end 97.25 84.3) (width 0.25) (layer F.Cu) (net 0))
 (segment (start 97.25 84.3) (end 92 89.55) (width 0.25) (layer F.Cu) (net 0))
 (via (at 100.45 81.1) (size 0.6) (drill 0.4) (layers F.Cu B.Cu) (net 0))
 (segment (start 91.75 85.05) (end 96.2 85.05) (width 0.25) (layer B.Cu) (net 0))
 (segment (start 96.2 85.05) (end 98.6 82.65) (width 0.25) (layer B.Cu) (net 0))
 (segment (start 98.6 82.65) (end 100.45 82.65) (width 0.25) (layer B.Cu) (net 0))
 (segment (start 93 88.25) (end 96.2 85.05) (width 0.25) (layer B.Cu) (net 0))
 (segment (start 91.75 88.25) (end 93 88.25) (width 0.25) (layer B.Cu) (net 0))
 (segment (start 96.5 81.1) (end 96.5 79.7) (width 0.25) (layer B.Cu) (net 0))
 (segment (start 91.984 75.184) (end 85.598 75.184) (width 0.25) (layer B.Cu) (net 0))
 (segment (start 96.5 79.7) (end 91.984 75.184) (width 0.25) (layer B.Cu) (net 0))
 (segment (start 95.7 81.1) (end 95.7 79.95) (width 0.25) (layer B.Cu) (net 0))
 (segment (start 93.474 77.724) (end 85.598 77.724) (width 0.25) (layer B.Cu) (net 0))
 (segment (start 95.7 79.95) (end 93.474 77.724) (width 0.25) (layer B.Cu) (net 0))
 (segment (start 94.9 81.1) (end 94.9 80.1) (width 0.25) (layer B.Cu) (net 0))
 (segment (start 86.962 78.9) (end 85.598 80.264) (width 0.25) (layer B.Cu) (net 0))
 (segment (start 93.7 78.9) (end 86.962 78.9) (width 0.25) (layer B.Cu) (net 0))
 (segment (start 94.9 80.1) (end 93.7 78.9) (width 0.25) (layer B.Cu) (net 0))
 (segment (start 94.1 81.1) (end 94.1 79.95) (width 0.25) (layer B.Cu) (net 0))
 (segment (start 88.902 79.5) (end 85.598 82.804) (width 0.25) (layer B.Cu) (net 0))
 (segment (start 93.65 79.5) (end 88.902 79.5) (width 0.25) (layer B.Cu) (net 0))
 (segment (start 94.1 79.95) (end 93.65 79.5) (width 0.25) (layer B.Cu) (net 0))
 (segment (start 93.3 81.1) (end 89.842 81.1) (width 0.25) (layer B.Cu) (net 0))
 (segment (start 89.842 81.1) (end 85.598 85.344) (width 0.25) (layer B.Cu) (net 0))
 (segment (start 91.75 82.65) (end 90.25 82.65) (width 0.25) (layer B.Cu) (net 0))
 (segment (start 87.95 85.532) (end 85.598 87.884) (width 0.25) (layer B.Cu) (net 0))
 (segment (start 87.95 84.95) (end 87.95 85.532) (width 0.25) (layer B.Cu) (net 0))
 (segment (start 90.25 82.65) (end 87.95 84.95) (width 0.25) (layer B.Cu) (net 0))
 (segment (start 91.75 83.45) (end 90.15 83.45) (width 0.25) (layer B.Cu) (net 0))
 (segment (start 88.45 87.572) (end 85.598 90.424) (width 0.25) (layer B.Cu) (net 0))
 (segment (start 88.45 85.15) (end 88.45 87.572) (width 0.25) (layer B.Cu) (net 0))
 (segment (start 90.15 83.45) (end 88.45 85.15) (width 0.25) (layer B.Cu) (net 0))
 (segment (start 91.75 84.25) (end 90.15 84.25) (width 0.25) (layer B.Cu) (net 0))
 (segment (start 89 89.562) (end 85.598 92.964) (width 0.25) (layer B.Cu) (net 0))
 (segment (start 89 85.4) (end 89 89.562) (width 0.25) (layer B.Cu) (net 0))
 (segment (start 90.15 84.25) (end 89 85.4) (width 0.25) (layer B.Cu) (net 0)))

